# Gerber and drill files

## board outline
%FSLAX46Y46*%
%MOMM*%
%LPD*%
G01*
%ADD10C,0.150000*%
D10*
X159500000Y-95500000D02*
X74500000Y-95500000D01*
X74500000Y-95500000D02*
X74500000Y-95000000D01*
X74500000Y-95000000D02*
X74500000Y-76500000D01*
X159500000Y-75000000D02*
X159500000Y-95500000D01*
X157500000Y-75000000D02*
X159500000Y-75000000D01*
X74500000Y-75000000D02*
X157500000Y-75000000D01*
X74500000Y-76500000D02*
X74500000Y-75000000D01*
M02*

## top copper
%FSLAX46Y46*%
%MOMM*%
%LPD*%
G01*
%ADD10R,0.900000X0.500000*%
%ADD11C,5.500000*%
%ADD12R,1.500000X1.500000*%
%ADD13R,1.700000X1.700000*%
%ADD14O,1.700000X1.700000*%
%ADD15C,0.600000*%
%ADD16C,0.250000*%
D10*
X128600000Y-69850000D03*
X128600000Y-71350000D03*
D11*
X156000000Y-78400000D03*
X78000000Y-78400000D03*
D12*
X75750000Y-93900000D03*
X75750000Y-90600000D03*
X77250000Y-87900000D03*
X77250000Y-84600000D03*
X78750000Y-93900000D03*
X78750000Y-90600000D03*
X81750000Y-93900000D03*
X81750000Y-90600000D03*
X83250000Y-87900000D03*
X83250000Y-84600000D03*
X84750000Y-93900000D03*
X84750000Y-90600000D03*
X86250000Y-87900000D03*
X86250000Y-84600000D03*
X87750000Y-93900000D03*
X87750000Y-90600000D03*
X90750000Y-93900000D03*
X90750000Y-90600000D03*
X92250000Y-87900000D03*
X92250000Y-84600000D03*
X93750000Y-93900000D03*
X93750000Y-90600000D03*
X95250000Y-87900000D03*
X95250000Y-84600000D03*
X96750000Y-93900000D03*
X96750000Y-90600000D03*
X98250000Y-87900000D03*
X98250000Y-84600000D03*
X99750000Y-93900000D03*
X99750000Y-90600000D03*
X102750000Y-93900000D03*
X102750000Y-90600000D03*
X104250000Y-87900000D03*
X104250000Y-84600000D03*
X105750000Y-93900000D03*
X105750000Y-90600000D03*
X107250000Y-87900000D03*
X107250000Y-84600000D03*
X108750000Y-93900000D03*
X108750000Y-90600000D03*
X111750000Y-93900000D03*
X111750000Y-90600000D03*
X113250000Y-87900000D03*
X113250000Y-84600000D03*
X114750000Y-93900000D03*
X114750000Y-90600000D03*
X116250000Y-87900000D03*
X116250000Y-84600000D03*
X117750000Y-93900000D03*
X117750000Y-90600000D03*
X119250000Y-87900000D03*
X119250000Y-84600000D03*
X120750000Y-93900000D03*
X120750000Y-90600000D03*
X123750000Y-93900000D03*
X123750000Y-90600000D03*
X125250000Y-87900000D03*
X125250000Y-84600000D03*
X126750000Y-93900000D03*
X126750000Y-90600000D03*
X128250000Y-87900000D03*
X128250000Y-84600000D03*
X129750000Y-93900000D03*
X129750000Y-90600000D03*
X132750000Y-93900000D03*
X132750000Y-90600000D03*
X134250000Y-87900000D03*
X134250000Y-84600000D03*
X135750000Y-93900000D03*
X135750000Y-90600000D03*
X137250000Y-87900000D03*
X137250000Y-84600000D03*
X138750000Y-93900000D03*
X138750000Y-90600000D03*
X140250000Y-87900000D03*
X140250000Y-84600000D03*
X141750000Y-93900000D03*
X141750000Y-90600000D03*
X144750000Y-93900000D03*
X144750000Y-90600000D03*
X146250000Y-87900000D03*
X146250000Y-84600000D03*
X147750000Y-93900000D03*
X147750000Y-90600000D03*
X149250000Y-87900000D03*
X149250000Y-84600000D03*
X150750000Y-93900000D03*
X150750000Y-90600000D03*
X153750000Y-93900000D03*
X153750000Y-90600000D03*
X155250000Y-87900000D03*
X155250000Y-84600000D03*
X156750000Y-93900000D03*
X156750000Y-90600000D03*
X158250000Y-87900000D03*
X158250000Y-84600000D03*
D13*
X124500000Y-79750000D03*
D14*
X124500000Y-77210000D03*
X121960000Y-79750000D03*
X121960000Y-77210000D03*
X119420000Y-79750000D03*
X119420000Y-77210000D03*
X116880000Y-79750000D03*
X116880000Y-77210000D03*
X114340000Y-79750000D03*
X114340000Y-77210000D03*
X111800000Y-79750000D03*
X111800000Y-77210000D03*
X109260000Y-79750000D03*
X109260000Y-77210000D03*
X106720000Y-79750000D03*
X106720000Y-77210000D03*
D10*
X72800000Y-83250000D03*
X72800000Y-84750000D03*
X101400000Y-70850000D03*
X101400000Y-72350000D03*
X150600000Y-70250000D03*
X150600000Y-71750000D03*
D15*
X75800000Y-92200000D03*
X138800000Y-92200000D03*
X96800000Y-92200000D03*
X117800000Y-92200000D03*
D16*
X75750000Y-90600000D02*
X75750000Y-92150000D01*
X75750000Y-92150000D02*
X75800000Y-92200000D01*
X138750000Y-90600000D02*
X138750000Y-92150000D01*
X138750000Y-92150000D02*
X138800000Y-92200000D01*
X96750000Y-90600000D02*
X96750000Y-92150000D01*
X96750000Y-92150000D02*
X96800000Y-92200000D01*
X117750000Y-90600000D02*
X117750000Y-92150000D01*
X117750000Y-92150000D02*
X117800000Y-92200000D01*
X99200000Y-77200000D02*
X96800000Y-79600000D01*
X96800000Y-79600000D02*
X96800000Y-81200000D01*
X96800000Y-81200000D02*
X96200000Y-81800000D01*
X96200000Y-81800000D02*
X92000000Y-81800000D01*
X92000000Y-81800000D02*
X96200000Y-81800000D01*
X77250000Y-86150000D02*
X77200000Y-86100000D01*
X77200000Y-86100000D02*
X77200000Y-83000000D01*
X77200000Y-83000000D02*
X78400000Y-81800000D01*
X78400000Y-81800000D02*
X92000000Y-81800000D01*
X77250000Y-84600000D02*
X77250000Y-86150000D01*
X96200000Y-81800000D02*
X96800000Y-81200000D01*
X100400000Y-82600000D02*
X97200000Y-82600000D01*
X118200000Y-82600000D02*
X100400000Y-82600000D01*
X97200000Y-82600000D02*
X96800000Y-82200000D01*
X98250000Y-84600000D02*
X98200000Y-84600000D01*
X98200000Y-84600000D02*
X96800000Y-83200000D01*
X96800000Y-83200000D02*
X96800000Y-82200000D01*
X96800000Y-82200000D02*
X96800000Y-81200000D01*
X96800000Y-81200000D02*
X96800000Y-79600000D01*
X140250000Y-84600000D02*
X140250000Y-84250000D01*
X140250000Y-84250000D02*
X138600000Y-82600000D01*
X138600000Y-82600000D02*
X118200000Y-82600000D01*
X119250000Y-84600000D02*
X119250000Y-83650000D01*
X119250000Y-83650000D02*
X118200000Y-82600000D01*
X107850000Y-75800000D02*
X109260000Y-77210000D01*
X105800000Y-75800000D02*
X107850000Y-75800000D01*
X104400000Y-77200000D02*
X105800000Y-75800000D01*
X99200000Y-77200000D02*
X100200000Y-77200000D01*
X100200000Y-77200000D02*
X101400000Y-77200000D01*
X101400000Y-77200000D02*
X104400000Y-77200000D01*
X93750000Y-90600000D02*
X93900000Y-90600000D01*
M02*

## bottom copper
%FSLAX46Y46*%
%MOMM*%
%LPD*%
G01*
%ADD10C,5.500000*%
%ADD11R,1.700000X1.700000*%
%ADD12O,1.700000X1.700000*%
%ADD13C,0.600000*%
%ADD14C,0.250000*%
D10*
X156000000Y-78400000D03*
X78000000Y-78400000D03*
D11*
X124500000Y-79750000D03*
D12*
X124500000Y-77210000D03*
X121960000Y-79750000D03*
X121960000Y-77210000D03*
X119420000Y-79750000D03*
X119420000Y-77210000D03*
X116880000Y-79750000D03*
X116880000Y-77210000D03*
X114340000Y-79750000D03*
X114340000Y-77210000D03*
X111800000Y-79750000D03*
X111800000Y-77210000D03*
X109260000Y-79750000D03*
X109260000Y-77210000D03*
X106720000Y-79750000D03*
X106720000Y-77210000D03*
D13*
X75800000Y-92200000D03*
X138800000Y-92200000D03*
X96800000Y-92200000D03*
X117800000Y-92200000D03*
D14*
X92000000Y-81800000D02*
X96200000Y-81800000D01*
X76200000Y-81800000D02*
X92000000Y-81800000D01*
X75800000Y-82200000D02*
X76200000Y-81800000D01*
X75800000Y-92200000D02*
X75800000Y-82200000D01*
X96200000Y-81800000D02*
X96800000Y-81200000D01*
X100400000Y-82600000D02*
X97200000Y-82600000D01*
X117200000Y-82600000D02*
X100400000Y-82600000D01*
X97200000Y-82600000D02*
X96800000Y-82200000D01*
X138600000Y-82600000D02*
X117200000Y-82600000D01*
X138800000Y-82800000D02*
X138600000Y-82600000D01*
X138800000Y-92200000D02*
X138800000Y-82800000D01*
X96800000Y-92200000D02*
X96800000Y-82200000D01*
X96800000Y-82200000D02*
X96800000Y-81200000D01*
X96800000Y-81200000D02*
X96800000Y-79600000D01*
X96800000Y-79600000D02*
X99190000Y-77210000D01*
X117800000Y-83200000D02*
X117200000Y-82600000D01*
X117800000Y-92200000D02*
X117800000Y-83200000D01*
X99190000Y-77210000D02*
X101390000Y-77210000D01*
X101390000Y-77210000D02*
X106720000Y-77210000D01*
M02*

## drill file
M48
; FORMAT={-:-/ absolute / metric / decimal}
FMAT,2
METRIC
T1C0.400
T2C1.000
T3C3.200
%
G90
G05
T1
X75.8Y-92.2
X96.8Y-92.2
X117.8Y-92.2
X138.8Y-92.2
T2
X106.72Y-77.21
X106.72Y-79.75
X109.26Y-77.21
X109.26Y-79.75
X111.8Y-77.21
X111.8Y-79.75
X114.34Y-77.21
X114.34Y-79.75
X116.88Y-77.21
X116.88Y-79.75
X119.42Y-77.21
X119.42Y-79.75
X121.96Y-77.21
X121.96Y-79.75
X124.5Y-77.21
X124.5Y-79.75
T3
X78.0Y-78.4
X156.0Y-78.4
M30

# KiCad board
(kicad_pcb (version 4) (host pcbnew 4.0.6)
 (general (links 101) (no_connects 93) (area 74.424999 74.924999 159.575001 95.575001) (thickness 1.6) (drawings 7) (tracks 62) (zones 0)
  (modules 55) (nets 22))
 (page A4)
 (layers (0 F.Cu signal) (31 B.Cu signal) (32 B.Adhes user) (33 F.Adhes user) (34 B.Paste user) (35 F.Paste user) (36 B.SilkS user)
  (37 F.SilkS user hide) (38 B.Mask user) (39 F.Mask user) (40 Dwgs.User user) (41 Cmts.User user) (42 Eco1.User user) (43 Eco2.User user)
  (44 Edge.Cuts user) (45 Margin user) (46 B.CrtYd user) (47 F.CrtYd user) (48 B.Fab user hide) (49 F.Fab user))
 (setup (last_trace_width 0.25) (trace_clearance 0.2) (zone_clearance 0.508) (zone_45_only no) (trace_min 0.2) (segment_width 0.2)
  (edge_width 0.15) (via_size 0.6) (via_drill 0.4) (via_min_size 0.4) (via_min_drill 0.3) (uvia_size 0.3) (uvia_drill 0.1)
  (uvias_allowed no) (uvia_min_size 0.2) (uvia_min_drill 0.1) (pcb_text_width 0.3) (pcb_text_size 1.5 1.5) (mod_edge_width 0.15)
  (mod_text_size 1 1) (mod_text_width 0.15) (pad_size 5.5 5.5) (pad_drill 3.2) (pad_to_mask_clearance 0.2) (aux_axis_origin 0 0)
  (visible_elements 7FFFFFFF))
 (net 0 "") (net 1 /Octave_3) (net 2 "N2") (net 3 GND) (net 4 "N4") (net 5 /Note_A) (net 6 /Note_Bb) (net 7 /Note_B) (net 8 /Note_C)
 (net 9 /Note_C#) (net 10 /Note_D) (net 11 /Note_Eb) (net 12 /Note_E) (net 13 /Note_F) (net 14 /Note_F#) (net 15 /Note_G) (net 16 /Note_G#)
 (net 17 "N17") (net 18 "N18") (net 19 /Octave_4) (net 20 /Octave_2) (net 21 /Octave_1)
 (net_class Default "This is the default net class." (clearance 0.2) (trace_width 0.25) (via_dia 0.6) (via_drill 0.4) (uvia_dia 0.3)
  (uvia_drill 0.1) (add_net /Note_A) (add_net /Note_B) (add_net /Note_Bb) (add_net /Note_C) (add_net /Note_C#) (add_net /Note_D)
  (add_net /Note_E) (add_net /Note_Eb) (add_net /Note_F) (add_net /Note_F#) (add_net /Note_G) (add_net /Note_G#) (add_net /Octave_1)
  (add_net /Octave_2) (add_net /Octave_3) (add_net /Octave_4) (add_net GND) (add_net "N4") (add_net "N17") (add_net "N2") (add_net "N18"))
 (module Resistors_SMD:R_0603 (layer F.Cu) (at 128.6 70.6 270)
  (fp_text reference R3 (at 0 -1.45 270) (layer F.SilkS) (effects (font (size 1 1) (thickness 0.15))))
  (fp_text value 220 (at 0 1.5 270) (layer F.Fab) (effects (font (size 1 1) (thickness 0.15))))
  (pad 1 smd rect (at -0.75 0 270) (size 0.5 0.9) (layers F.Cu F.Paste F.Mask) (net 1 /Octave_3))
  (pad 2 smd rect (at 0.75 0 270) (size 0.5 0.9) (layers F.Cu F.Paste F.Mask) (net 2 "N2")))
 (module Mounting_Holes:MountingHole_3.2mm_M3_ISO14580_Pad (layer F.Cu) (at 156 78.4)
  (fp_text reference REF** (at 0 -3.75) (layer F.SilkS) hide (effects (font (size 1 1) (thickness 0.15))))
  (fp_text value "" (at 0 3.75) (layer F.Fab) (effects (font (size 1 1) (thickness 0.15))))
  (pad 1 thru_hole circle (at 0 0) (size 5.5 5.5) (drill 3.2) (layers *.Cu *.Mask) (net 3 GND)))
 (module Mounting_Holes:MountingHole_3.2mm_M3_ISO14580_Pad (layer F.Cu) (at 78 78.4)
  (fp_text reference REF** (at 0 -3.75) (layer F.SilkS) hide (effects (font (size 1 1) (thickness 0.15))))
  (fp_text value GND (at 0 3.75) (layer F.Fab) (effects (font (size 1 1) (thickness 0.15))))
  (pad 1 thru_hole circle (at 0 0) (size 5.5 5.5) (drill 3.2) (layers *.Cu *.Mask) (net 3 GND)))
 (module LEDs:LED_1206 (layer F.Cu) (at 75.75 92.25 270)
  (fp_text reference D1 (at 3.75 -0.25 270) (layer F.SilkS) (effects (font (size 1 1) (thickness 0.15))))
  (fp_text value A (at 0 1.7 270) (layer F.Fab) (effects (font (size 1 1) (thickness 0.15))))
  (pad 2 smd rect (at 1.65 0 90) (size 1.5 1.5) (layers F.Cu F.Paste F.Mask) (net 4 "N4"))
  (pad 1 smd rect (at -1.65 0 90) (size 1.5 1.5) (layers F.Cu F.Paste F.Mask) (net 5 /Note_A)))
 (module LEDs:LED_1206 (layer F.Cu) (at 77.25 86.25 270)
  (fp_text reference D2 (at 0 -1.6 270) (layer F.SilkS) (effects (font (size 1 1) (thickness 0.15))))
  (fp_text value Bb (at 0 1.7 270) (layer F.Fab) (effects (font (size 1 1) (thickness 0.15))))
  (pad 2 smd rect (at 1.65 0 90) (size 1.5 1.5) (layers F.Cu F.Paste F.Mask) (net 4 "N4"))
  (pad 1 smd rect (at -1.65 0 90) (size 1.5 1.5) (layers F.Cu F.Paste F.Mask) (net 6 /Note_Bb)))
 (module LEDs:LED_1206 (layer F.Cu) (at 78.75 92.25 270)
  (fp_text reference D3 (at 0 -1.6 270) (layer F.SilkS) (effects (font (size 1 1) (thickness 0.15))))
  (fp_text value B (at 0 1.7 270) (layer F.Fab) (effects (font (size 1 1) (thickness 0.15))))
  (pad 2 smd rect (at 1.65 0 90) (size 1.5 1.5) (layers F.Cu F.Paste F.Mask) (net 4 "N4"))
  (pad 1 smd rect (at -1.65 0 90) (size 1.5 1.5) (layers F.Cu F.Paste F.Mask) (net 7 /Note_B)))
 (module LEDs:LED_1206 (layer F.Cu) (at 81.75 92.25 270)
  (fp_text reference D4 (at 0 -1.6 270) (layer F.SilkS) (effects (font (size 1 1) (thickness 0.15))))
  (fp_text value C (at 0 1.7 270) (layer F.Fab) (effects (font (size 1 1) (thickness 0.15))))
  (pad 2 smd rect (at 1.65 0 90) (size 1.5 1.5) (layers F.Cu F.Paste F.Mask) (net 4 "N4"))
  (pad 1 smd rect (at -1.65 0 90) (size 1.5 1.5) (layers F.Cu F.Paste F.Mask) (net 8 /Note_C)))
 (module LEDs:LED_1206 (layer F.Cu) (at 83.25 86.25 270)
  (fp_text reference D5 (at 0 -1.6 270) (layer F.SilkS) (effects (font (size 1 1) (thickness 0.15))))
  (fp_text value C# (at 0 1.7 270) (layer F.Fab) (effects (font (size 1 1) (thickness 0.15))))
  (pad 2 smd rect (at 1.65 0 90) (size 1.5 1.5) (layers F.Cu F.Paste F.Mask) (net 4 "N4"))
  (pad 1 smd rect (at -1.65 0 90) (size 1.5 1.5) (layers F.Cu F.Paste F.Mask) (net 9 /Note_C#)))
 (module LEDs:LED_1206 (layer F.Cu) (at 84.75 92.25 270)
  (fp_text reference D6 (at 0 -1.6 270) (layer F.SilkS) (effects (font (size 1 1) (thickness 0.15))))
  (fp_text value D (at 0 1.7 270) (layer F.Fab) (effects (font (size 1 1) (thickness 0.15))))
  (pad 2 smd rect (at 1.65 0 90) (size 1.5 1.5) (layers F.Cu F.Paste F.Mask) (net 4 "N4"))
  (pad 1 smd rect (at -1.65 0 90) (size 1.5 1.5) (layers F.Cu F.Paste F.Mask) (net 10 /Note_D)))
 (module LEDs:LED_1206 (layer F.Cu) (at 86.25 86.25 270)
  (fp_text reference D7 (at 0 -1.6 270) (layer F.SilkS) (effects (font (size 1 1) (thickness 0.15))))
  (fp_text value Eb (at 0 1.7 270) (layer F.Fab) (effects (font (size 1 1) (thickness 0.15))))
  (pad 2 smd rect (at 1.65 0 90) (size 1.5 1.5) (layers F.Cu F.Paste F.Mask) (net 4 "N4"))
  (pad 1 smd rect (at -1.65 0 90) (size 1.5 1.5) (layers F.Cu F.Paste F.Mask) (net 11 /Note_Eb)))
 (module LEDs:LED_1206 (layer F.Cu) (at 87.75 92.25 270)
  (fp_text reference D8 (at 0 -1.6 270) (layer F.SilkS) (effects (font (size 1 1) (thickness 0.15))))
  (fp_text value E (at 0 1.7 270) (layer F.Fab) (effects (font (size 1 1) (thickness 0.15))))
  (pad 2 smd rect (at 1.65 0 90) (size 1.5 1.5) (layers F.Cu F.Paste F.Mask) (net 4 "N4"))
  (pad 1 smd rect (at -1.65 0 90) (size 1.5 1.5) (layers F.Cu F.Paste F.Mask) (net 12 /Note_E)))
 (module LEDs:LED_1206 (layer F.Cu) (at 90.75 92.25 270)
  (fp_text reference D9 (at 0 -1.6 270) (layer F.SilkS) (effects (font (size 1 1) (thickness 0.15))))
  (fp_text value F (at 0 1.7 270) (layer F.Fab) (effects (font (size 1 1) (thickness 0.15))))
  (pad 2 smd rect (at 1.65 0 90) (size 1.5 1.5) (layers F.Cu F.Paste F.Mask) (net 4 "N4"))
  (pad 1 smd rect (at -1.65 0 90) (size 1.5 1.5) (layers F.Cu F.Paste F.Mask) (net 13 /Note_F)))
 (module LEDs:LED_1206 (layer F.Cu) (at 92.25 86.25 270)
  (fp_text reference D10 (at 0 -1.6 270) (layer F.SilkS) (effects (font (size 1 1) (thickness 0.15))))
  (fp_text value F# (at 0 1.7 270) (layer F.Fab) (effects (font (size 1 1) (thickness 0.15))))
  (pad 2 smd rect (at 1.65 0 90) (size 1.5 1.5) (layers F.Cu F.Paste F.Mask) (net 4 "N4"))
  (pad 1 smd rect (at -1.65 0 90) (size 1.5 1.5) (layers F.Cu F.Paste F.Mask) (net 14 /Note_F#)))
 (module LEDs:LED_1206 (layer F.Cu) (at 93.75 92.25 270)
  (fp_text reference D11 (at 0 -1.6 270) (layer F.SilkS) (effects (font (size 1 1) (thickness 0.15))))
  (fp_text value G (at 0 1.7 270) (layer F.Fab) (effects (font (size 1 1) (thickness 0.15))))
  (pad 2 smd rect (at 1.65 0 90) (size 1.5 1.5) (layers F.Cu F.Paste F.Mask) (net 4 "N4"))
  (pad 1 smd rect (at -1.65 0 90) (size 1.5 1.5) (layers F.Cu F.Paste F.Mask) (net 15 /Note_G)))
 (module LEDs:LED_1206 (layer F.Cu) (at 95.25 86.25 270)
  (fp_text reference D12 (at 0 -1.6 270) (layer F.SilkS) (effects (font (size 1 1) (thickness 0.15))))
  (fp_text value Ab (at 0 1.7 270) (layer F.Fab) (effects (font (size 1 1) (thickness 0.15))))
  (pad 2 smd rect (at 1.65 0 90) (size 1.5 1.5) (layers F.Cu F.Paste F.Mask) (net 4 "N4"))
  (pad 1 smd rect (at -1.65 0 90) (size 1.5 1.5) (layers F.Cu F.Paste F.Mask) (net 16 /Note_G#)))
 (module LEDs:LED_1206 (layer F.Cu) (at 96.75 92.25 270)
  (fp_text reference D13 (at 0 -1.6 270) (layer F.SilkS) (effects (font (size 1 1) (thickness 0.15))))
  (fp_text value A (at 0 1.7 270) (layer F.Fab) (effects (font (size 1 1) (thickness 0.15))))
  (pad 2 smd rect (at 1.65 0 90) (size 1.5 1.5) (layers F.Cu F.Paste F.Mask) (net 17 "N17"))
  (pad 1 smd rect (at -1.65 0 90) (size 1.5 1.5) (layers F.Cu F.Paste F.Mask) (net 5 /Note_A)))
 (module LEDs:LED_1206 (layer F.Cu) (at 98.25 86.25 270)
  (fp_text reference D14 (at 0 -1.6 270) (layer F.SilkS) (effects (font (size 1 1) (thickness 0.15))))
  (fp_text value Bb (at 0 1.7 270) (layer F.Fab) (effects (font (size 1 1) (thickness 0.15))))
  (pad 2 smd rect (at 1.65 0 90) (size 1.5 1.5) (layers F.Cu F.Paste F.Mask) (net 17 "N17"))
  (pad 1 smd rect (at -1.65 0 90) (size 1.5 1.5) (layers F.Cu F.Paste F.Mask) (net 6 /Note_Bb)))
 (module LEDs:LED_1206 (layer F.Cu) (at 99.75 92.25 270)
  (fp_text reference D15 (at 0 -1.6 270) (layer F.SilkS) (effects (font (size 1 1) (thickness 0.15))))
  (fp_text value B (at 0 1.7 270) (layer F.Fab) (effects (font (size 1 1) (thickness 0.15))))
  (pad 2 smd rect (at 1.65 0 90) (size 1.5 1.5) (layers F.Cu F.Paste F.Mask) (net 17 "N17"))
  (pad 1 smd rect (at -1.65 0 90) (size 1.5 1.5) (layers F.Cu F.Paste F.Mask) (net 7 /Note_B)))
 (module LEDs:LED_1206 (layer F.Cu) (at 102.75 92.25 270)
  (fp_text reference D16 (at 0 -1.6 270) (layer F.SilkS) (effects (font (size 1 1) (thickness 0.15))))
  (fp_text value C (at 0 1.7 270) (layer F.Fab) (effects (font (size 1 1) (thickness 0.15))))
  (pad 2 smd rect (at 1.65 0 90) (size 1.5 1.5) (layers F.Cu F.Paste F.Mask) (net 17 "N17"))
  (pad 1 smd rect (at -1.65 0 90) (size 1.5 1.5) (layers F.Cu F.Paste F.Mask) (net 8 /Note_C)))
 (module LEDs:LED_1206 (layer F.Cu) (at 104.25 86.25 270)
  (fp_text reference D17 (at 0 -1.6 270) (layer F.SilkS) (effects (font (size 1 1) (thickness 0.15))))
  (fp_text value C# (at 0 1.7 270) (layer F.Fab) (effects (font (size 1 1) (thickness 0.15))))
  (pad 2 smd rect (at 1.65 0 90) (size 1.5 1.5) (layers F.Cu F.Paste F.Mask) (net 17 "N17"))
  (pad 1 smd rect (at -1.65 0 90) (size 1.5 1.5) (layers F.Cu F.Paste F.Mask) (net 9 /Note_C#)))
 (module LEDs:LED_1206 (layer F.Cu) (at 105.75 92.25 270)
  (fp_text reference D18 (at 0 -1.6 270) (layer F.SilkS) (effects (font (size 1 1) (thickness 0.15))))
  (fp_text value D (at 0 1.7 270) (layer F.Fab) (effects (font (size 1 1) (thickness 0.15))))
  (pad 2 smd rect (at 1.65 0 90) (size 1.5 1.5) (layers F.Cu F.Paste F.Mask) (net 17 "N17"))
  (pad 1 smd rect (at -1.65 0 90) (size 1.5 1.5) (layers F.Cu F.Paste F.Mask) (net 10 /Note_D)))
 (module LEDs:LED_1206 (layer F.Cu) (at 107.25 86.25 270)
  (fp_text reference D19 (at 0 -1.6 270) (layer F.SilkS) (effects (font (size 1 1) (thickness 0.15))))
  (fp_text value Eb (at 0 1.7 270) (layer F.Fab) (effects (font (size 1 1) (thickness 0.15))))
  (pad 2 smd rect (at 1.65 0 90) (size 1.5 1.5) (layers F.Cu F.Paste F.Mask) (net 17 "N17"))
  (pad 1 smd rect (at -1.65 0 90) (size 1.5 1.5) (layers F.Cu F.Paste F.Mask) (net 11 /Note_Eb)))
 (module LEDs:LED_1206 (layer F.Cu) (at 108.75 92.25 270)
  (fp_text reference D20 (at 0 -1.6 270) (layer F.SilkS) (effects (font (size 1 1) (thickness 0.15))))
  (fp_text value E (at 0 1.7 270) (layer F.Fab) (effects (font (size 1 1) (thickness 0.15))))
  (pad 2 smd rect (at 1.65 0 90) (size 1.5 1.5) (layers F.Cu F.Paste F.Mask) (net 17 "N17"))
  (pad 1 smd rect (at -1.65 0 90) (size 1.5 1.5) (layers F.Cu F.Paste F.Mask) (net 12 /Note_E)))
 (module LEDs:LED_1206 (layer F.Cu) (at 111.75 92.25 270)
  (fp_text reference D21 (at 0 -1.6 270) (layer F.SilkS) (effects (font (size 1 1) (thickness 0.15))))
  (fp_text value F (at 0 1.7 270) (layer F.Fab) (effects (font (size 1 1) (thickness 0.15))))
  (pad 2 smd rect (at 1.65 0 90) (size 1.5 1.5) (layers F.Cu F.Paste F.Mask) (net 17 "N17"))
  (pad 1 smd rect (at -1.65 0 90) (size 1.5 1.5) (layers F.Cu F.Paste F.Mask) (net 13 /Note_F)))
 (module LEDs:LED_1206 (layer F.Cu) (at 113.25 86.25 270)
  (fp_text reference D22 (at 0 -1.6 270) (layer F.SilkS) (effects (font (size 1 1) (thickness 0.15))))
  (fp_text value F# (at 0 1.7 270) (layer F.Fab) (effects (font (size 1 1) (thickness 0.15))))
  (pad 2 smd rect (at 1.65 0 90) (size 1.5 1.5) (layers F.Cu F.Paste F.Mask) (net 17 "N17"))
  (pad 1 smd rect (at -1.65 0 90) (size 1.5 1.5) (layers F.Cu F.Paste F.Mask) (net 14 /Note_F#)))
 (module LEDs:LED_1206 (layer F.Cu) (at 114.75 92.25 270)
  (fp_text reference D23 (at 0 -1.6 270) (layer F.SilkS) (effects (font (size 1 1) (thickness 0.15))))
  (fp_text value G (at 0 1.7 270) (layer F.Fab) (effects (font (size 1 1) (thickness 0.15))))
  (pad 2 smd rect (at 1.65 0 90) (size 1.5 1.5) (layers F.Cu F.Paste F.Mask) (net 17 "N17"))
  (pad 1 smd rect (at -1.65 0 90) (size 1.5 1.5) (layers F.Cu F.Paste F.Mask) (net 15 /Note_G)))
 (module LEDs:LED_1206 (layer F.Cu) (at 116.25 86.25 270)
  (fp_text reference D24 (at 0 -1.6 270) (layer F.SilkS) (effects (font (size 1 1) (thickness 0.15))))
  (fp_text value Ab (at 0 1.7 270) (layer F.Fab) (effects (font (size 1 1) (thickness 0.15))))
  (pad 2 smd rect (at 1.65 0 90) (size 1.5 1.5) (layers F.Cu F.Paste F.Mask) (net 17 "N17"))
  (pad 1 smd rect (at -1.65 0 90) (size 1.5 1.5) (layers F.Cu F.Paste F.Mask) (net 16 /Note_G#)))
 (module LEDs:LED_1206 (layer F.Cu) (at 117.75 92.25 270)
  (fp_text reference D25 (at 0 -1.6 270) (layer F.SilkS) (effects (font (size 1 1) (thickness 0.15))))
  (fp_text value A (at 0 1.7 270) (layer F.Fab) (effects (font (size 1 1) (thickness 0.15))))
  (pad 2 smd rect (at 1.65 0 90) (size 1.5 1.5) (layers F.Cu F.Paste F.Mask) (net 2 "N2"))
  (pad 1 smd rect (at -1.65 0 90) (size 1.5 1.5) (layers F.Cu F.Paste F.Mask) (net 5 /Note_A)))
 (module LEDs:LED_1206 (layer F.Cu) (at 119.25 86.25 270)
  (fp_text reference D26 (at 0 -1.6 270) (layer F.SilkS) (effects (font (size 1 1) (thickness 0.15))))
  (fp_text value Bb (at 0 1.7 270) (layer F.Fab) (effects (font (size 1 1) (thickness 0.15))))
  (pad 2 smd rect (at 1.65 0 90) (size 1.5 1.5) (layers F.Cu F.Paste F.Mask) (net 2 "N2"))
  (pad 1 smd rect (at -1.65 0 90) (size 1.5 1.5) (layers F.Cu F.Paste F.Mask) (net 6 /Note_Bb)))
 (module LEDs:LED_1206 (layer F.Cu) (at 120.75 92.25 270)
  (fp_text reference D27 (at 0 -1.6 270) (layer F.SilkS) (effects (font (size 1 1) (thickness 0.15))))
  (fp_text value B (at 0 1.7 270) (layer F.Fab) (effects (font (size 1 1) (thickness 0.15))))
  (pad 2 smd rect (at 1.65 0 90) (size 1.5 1.5) (layers F.Cu F.Paste F.Mask) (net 2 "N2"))
  (pad 1 smd rect (at -1.65 0 90) (size 1.5 1.5) (layers F.Cu F.Paste F.Mask) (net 7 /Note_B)))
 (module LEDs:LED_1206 (layer F.Cu) (at 123.75 92.25 270)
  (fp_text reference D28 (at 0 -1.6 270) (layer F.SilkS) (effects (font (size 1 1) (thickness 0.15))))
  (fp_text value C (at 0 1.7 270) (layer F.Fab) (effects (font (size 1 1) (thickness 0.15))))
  (pad 2 smd rect (at 1.65 0 90) (size 1.5 1.5) (layers F.Cu F.Paste F.Mask) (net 2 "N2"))
  (pad 1 smd rect (at -1.65 0 90) (size 1.5 1.5) (layers F.Cu F.Paste F.Mask) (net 8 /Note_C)))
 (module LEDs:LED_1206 (layer F.Cu) (at 125.25 86.25 270)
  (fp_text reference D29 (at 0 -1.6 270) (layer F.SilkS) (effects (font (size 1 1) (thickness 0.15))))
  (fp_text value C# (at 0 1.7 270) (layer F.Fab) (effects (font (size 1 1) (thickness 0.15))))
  (pad 2 smd rect (at 1.65 0 90) (size 1.5 1.5) (layers F.Cu F.Paste F.Mask) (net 2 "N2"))
  (pad 1 smd rect (at -1.65 0 90) (size 1.5 1.5) (layers F.Cu F.Paste F.Mask) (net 9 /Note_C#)))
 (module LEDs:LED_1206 (layer F.Cu) (at 126.75 92.25 270)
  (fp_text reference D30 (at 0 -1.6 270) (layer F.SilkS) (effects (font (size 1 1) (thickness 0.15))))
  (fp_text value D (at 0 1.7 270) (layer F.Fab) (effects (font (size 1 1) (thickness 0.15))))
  (pad 2 smd rect (at 1.65 0 90) (size 1.5 1.5) (layers F.Cu F.Paste F.Mask) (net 2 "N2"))
  (pad 1 smd rect (at -1.65 0 90) (size 1.5 1.5) (layers F.Cu F.Paste F.Mask) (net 10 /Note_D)))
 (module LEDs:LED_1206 (layer F.Cu) (at 128.25 86.25 270)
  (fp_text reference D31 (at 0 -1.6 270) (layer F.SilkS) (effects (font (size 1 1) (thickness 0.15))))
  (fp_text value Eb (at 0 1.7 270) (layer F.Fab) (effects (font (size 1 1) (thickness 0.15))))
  (pad 2 smd rect (at 1.65 0 90) (size 1.5 1.5) (layers F.Cu F.Paste F.Mask) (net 2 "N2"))
  (pad 1 smd rect (at -1.65 0 90) (size 1.5 1.5) (layers F.Cu F.Paste F.Mask) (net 11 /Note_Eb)))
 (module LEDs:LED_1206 (layer F.Cu) (at 129.75 92.25 270)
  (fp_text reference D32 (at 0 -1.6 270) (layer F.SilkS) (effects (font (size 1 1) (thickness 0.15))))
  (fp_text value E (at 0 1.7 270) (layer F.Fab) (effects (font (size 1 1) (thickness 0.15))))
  (pad 2 smd rect (at 1.65 0 90) (size 1.5 1.5) (layers F.Cu F.Paste F.Mask) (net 2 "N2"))
  (pad 1 smd rect (at -1.65 0 90) (size 1.5 1.5) (layers F.Cu F.Paste F.Mask) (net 12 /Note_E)))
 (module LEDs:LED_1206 (layer F.Cu) (at 132.75 92.25 270)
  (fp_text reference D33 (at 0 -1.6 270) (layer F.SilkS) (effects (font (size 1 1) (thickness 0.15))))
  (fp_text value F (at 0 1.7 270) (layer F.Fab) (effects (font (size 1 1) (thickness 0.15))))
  (pad 2 smd rect (at 1.65 0 90) (size 1.5 1.5) (layers F.Cu F.Paste F.Mask) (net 2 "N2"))
  (pad 1 smd rect (at -1.65 0 90) (size 1.5 1.5) (layers F.Cu F.Paste F.Mask) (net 13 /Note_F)))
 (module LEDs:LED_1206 (layer F.Cu) (at 134.25 86.25 270)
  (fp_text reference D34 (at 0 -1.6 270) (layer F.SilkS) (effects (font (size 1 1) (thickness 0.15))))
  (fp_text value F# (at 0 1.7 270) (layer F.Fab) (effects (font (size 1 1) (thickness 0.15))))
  (pad 2 smd rect (at 1.65 0 90) (size 1.5 1.5) (layers F.Cu F.Paste F.Mask) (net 2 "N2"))
  (pad 1 smd rect (at -1.65 0 90) (size 1.5 1.5) (layers F.Cu F.Paste F.Mask) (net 14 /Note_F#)))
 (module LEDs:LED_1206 (layer F.Cu) (at 135.75 92.25 270)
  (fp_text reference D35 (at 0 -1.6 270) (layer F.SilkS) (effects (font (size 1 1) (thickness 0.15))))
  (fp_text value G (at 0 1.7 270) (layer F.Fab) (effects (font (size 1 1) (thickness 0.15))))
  (pad 2 smd rect (at 1.65 0 90) (size 1.5 1.5) (layers F.Cu F.Paste F.Mask) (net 2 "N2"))
  (pad 1 smd rect (at -1.65 0 90) (size 1.5 1.5) (layers F.Cu F.Paste F.Mask) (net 15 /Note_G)))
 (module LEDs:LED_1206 (layer F.Cu) (at 137.25 86.25 270)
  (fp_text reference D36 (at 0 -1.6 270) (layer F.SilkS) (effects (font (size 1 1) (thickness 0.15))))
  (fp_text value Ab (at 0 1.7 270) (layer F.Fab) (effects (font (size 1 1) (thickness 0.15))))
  (pad 2 smd rect (at 1.65 0 90) (size 1.5 1.5) (layers F.Cu F.Paste F.Mask) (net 2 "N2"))
  (pad 1 smd rect (at -1.65 0 90) (size 1.5 1.5) (layers F.Cu F.Paste F.Mask) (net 16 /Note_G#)))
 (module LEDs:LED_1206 (layer F.Cu) (at 138.75 92.25 270)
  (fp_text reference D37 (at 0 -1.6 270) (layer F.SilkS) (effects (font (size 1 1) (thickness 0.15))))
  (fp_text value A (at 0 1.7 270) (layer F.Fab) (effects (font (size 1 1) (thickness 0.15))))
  (pad 2 smd rect (at 1.65 0 90) (size 1.5 1.5) (layers F.Cu F.Paste F.Mask) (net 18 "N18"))
  (pad 1 smd rect (at -1.65 0 90) (size 1.5 1.5) (layers F.Cu F.Paste F.Mask) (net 5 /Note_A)))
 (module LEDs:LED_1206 (layer F.Cu) (at 140.25 86.25 270)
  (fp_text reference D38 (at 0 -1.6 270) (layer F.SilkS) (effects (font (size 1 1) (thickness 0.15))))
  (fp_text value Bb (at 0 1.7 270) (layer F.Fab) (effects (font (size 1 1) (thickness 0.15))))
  (pad 2 smd rect (at 1.65 0 90) (size 1.5 1.5) (layers F.Cu F.Paste F.Mask) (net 18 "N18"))
  (pad 1 smd rect (at -1.65 0 90) (size 1.5 1.5) (layers F.Cu F.Paste F.Mask) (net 6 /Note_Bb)))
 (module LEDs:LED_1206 (layer F.Cu) (at 141.75 92.25 270)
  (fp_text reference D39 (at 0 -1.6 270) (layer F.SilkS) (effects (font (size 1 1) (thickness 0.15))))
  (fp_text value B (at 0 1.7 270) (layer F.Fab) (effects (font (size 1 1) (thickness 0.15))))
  (pad 2 smd rect (at 1.65 0 90) (size 1.5 1.5) (layers F.Cu F.Paste F.Mask) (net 18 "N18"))
  (pad 1 smd rect (at -1.65 0 90) (size 1.5 1.5) (layers F.Cu F.Paste F.Mask) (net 7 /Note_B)))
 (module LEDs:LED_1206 (layer F.Cu) (at 144.75 92.25 270)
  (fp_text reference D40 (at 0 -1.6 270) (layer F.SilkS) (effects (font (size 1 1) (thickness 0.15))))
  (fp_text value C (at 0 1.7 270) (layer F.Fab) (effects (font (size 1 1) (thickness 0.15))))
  (pad 2 smd rect (at 1.65 0 90) (size 1.5 1.5) (layers F.Cu F.Paste F.Mask) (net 18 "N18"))
  (pad 1 smd rect (at -1.65 0 90) (size 1.5 1.5) (layers F.Cu F.Paste F.Mask) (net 8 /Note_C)))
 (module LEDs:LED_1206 (layer F.Cu) (at 146.25 86.25 270)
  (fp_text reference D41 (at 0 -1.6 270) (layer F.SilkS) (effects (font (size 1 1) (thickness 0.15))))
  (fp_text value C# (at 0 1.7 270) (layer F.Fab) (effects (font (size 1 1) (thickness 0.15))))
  (pad 2 smd rect (at 1.65 0 90) (size 1.5 1.5) (layers F.Cu F.Paste F.Mask) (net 18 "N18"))
  (pad 1 smd rect (at -1.65 0 90) (size 1.5 1.5) (layers F.Cu F.Paste F.Mask) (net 9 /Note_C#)))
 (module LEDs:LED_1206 (layer F.Cu) (at 147.75 92.25 270)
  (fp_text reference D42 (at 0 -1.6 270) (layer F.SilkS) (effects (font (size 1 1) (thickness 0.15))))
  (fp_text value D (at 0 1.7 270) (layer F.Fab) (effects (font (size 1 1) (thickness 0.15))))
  (pad 2 smd rect (at 1.65 0 90) (size 1.5 1.5) (layers F.Cu F.Paste F.Mask) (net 18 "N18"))
  (pad 1 smd rect (at -1.65 0 90) (size 1.5 1.5) (layers F.Cu F.Paste F.Mask) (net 10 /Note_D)))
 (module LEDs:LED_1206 (layer F.Cu) (at 149.25 86.25 270)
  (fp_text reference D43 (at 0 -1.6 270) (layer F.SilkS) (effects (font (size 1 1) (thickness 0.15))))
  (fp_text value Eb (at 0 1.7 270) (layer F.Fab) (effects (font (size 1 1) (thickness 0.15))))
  (pad 2 smd rect (at 1.65 0 90) (size 1.5 1.5) (layers F.Cu F.Paste F.Mask) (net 18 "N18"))
  (pad 1 smd rect (at -1.65 0 90) (size 1.5 1.5) (layers F.Cu F.Paste F.Mask) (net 11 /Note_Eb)))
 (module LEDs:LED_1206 (layer F.Cu) (at 150.75 92.25 270)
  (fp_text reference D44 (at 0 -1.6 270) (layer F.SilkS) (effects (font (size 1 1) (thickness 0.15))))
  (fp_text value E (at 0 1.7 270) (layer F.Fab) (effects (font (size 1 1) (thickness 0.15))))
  (pad 2 smd rect (at 1.65 0 90) (size 1.5 1.5) (layers F.Cu F.Paste F.Mask) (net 18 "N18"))
  (pad 1 smd rect (at -1.65 0 90) (size 1.5 1.5) (layers F.Cu F.Paste F.Mask) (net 12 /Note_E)))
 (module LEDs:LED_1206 (layer F.Cu) (at 153.75 92.25 270)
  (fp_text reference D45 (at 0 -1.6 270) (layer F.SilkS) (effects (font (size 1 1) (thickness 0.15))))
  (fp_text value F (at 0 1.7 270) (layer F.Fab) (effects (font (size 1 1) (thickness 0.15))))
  (pad 2 smd rect (at 1.65 0 90) (size 1.5 1.5) (layers F.Cu F.Paste F.Mask) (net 18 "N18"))
  (pad 1 smd rect (at -1.65 0 90) (size 1.5 1.5) (layers F.Cu F.Paste F.Mask) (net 13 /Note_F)))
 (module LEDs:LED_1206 (layer F.Cu) (at 155.25 86.25 270)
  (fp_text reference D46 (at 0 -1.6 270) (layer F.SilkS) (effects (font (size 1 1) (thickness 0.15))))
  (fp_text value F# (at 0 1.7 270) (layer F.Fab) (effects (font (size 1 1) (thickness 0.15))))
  (pad 2 smd rect (at 1.65 0 90) (size 1.5 1.5) (layers F.Cu F.Paste F.Mask) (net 18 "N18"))
  (pad 1 smd rect (at -1.65 0 90) (size 1.5 1.5) (layers F.Cu F.Paste F.Mask) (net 14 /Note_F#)))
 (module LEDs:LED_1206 (layer F.Cu) (at 156.75 92.25 270)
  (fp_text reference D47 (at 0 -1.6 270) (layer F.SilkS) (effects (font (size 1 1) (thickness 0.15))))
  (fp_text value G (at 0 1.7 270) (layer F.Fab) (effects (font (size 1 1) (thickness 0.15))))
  (pad 2 smd rect (at 1.65 0 90) (size 1.5 1.5) (layers F.Cu F.Paste F.Mask) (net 18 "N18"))
  (pad 1 smd rect (at -1.65 0 90) (size 1.5 1.5) (layers F.Cu F.Paste F.Mask) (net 15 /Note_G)))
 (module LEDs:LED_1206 (layer F.Cu) (at 158.25 86.25 270)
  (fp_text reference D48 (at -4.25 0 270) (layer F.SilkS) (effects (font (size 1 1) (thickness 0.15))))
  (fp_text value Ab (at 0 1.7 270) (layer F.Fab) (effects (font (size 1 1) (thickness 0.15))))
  (pad 2 smd rect (at 1.65 0 90) (size 1.5 1.5) (layers F.Cu F.Paste F.Mask) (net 18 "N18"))
  (pad 1 smd rect (at -1.65 0 90) (size 1.5 1.5) (layers F.Cu F.Paste F.Mask) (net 16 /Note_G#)))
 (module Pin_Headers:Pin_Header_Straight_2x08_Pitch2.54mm (layer B.Cu) (at 124.5 79.75 90)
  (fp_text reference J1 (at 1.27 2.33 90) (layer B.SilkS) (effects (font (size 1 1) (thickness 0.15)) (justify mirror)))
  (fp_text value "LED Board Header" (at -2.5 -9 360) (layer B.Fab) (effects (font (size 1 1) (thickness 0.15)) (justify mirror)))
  (pad 1 thru_hole rect (at 0 0 90) (size 1.7 1.7) (drill 1) (layers *.Cu *.Mask) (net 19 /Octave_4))
  (pad 2 thru_hole oval (at 2.54 0 90) (size 1.7 1.7) (drill 1) (layers *.Cu *.Mask) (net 12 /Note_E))
  (pad 3 thru_hole oval (at 0 -2.54 90) (size 1.7 1.7) (drill 1) (layers *.Cu *.Mask) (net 1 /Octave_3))
  (pad 4 thru_hole oval (at 2.54 -2.54 90) (size 1.7 1.7) (drill 1) (layers *.Cu *.Mask) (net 11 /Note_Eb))
  (pad 5 thru_hole oval (at 0 -5.08 90) (size 1.7 1.7) (drill 1) (layers *.Cu *.Mask) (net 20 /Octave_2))
  (pad 6 thru_hole oval (at 2.54 -5.08 90) (size 1.7 1.7) (drill 1) (layers *.Cu *.Mask) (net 10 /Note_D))
  (pad 7 thru_hole oval (at 0 -7.62 90) (size 1.7 1.7) (drill 1) (layers *.Cu *.Mask) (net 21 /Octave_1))
  (pad 8 thru_hole oval (at 2.54 -7.62 90) (size 1.7 1.7) (drill 1) (layers *.Cu *.Mask) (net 9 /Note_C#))
  (pad 9 thru_hole oval (at 0 -10.16 90) (size 1.7 1.7) (drill 1) (layers *.Cu *.Mask) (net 16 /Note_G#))
  (pad 10 thru_hole oval (at 2.54 -10.16 90) (size 1.7 1.7) (drill 1) (layers *.Cu *.Mask) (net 8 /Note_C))
  (pad 11 thru_hole oval (at 0 -12.7 90) (size 1.7 1.7) (drill 1) (layers *.Cu *.Mask) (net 15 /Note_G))
  (pad 12 thru_hole oval (at 2.54 -12.7 90) (size 1.7 1.7) (drill 1) (layers *.Cu *.Mask) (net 7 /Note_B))
  (pad 13 thru_hole oval (at 0 -15.24 90) (size 1.7 1.7) (drill 1) (layers *.Cu *.Mask) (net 14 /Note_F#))
  (pad 14 thru_hole oval (at 2.54 -15.24 90) (size 1.7 1.7) (drill 1) (layers *.Cu *.Mask) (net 6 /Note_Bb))
  (pad 15 thru_hole oval (at 0 -17.78 90) (size 1.7 1.7) (drill 1) (layers *.Cu *.Mask) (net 13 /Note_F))
  (pad 16 thru_hole oval (at 2.54 -17.78 90) (size 1.7 1.7) (drill 1) (layers *.Cu *.Mask) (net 5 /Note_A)))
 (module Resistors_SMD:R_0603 (layer F.Cu) (at 72.8 84 270)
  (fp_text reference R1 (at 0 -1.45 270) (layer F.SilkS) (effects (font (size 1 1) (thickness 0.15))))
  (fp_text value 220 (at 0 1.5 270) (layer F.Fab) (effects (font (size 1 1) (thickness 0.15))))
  (pad 1 smd rect (at -0.75 0 270) (size 0.5 0.9) (layers F.Cu F.Paste F.Mask) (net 21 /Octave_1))
  (pad 2 smd rect (at 0.75 0 270) (size 0.5 0.9) (layers F.Cu F.Paste F.Mask) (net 4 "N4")))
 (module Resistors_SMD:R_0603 (layer F.Cu) (at 101.4 71.6 270)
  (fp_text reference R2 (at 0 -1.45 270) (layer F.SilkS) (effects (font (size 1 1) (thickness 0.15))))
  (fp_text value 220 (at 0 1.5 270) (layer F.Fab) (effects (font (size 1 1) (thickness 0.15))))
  (pad 1 smd rect (at -0.75 0 270) (size 0.5 0.9) (layers F.Cu F.Paste F.Mask) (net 20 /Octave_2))
  (pad 2 smd rect (at 0.75 0 270) (size 0.5 0.9) (layers F.Cu F.Paste F.Mask) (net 17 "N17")))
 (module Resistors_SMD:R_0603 (layer F.Cu) (at 150.6 71 270)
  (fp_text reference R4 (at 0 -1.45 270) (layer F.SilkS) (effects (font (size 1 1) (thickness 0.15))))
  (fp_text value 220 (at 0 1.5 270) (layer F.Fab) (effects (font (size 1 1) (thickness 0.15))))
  (pad 1 smd rect (at -0.75 0 270) (size 0.5 0.9) (layers F.Cu F.Paste F.Mask) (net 19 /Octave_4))
  (pad 2 smd rect (at 0.75 0 270) (size 0.5 0.9) (layers F.Cu F.Paste F.Mask) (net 18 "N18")))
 (gr_line (start 159.5 95.5) (end 74.5 95.5) (angle 90) (layer Edge.Cuts) (width 0.15))
 (gr_line (start 74.5 95.5) (end 74.5 95) (angle 90) (layer Edge.Cuts) (width 0.15))
 (gr_line (start 74.5 95) (end 74.5 76.5) (angle 90) (layer Edge.Cuts) (width 0.15))
 (gr_line (start 159.5 75) (end 159.5 95.5) (angle 90) (layer Edge.Cuts) (width 0.15))
 (gr_line (start 157.5 75) (end 159.5 75) (angle 90) (layer Edge.Cuts) (width 0.15))
 (gr_line (start 74.5 75) (end 157.5 75) (angle 90) (layer Edge.Cuts) (width 0.15))
 (gr_line (start 74.5 76.5) (end 74.5 75) (angle 90) (layer Edge.Cuts) (width 0.15))
 (segment (start 92 81.8) (end 96.2 81.8) (width 0.25) (layer B.Cu) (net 5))
 (segment (start 75.75 90.6) (end 75.75 92.15) (width 0.25) (layer F.Cu) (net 5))
 (segment (start 76.2 81.8) (end 92 81.8) (width 0.25) (layer B.Cu) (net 5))
 (segment (start 75.8 82.2) (end 76.2 81.8) (width 0.25) (layer B.Cu) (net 5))
 (segment (start 75.8 92.2) (end 75.8 82.2) (width 0.25) (layer B.Cu) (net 5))
 (via (at 75.8 92.2) (size 0.6) (drill 0.4) (layers F.Cu B.Cu) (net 5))
 (segment (start 75.75 92.15) (end 75.8 92.2) (width 0.25) (layer F.Cu) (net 5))
 (segment (start 96.2 81.8) (end 96.8 81.2) (width 0.25) (layer B.Cu) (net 5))
 (segment (start 100.4 82.6) (end 97.2 82.6) (width 0.25) (layer B.Cu) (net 5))
 (segment (start 117.2 82.6) (end 100.4 82.6) (width 0.25) (layer B.Cu) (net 5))
 (segment (start 97.2 82.6) (end 96.8 82.2) (width 0.25) (layer B.Cu) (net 5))
 (segment (start 138.75 90.6) (end 138.75 92.15) (width 0.25) (layer F.Cu) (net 5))
 (segment (start 138.6 82.6) (end 117.2 82.6) (width 0.25) (layer B.Cu) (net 5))
 (segment (start 138.8 82.8) (end 138.6 82.6) (width 0.25) (layer B.Cu) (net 5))
 (segment (start 138.8 92.2) (end 138.8 82.8) (width 0.25) (layer B.Cu) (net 5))
 (via (at 138.8 92.2) (size 0.6) (drill 0.4) (layers F.Cu B.Cu) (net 5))
 (segment (start 138.75 92.15) (end 138.8 92.2) (width 0.25) (layer F.Cu) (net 5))
 (segment (start 96.8 92.2) (end 96.8 82.2) (width 0.25) (layer B.Cu) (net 5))
 (segment (start 96.75 90.6) (end 96.75 92.15) (width 0.25) (layer F.Cu) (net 5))
 (via (at 96.8 92.2) (size 0.6) (drill 0.4) (layers F.Cu B.Cu) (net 5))
 (segment (start 96.75 92.15) (end 96.8 92.2) (width 0.25) (layer F.Cu) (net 5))
 (segment (start 96.8 82.2) (end 96.8 81.2) (width 0.25) (layer B.Cu) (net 5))
 (segment (start 96.8 81.2) (end 96.8 79.6) (width 0.25) (layer B.Cu) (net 5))
 (segment (start 96.8 79.6) (end 99.19 77.21) (width 0.25) (layer B.Cu) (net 5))
 (segment (start 117.75 90.6) (end 117.75 92.15) (width 0.25) (layer F.Cu) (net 5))
 (segment (start 117.8 83.2) (end 117.2 82.6) (width 0.25) (layer B.Cu) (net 5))
 (segment (start 117.8 92.2) (end 117.8 83.2) (width 0.25) (layer B.Cu) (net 5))
 (via (at 117.8 92.2) (size 0.6) (drill 0.4) (layers F.Cu B.Cu) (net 5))
 (segment (start 117.75 92.15) (end 117.8 92.2) (width 0.25) (layer F.Cu) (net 5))
 (segment (start 99.19 77.21) (end 101.39 77.21) (width 0.25) (layer B.Cu) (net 5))
 (segment (start 101.39 77.21) (end 106.72 77.21) (width 0.25) (layer B.Cu) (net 5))
 (segment (start 99.2 77.2) (end 96.8 79.6) (width 0.25) (layer F.Cu) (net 6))
 (segment (start 96.8 79.6) (end 96.8 81.2) (width 0.25) (layer F.Cu) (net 6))
 (segment (start 96.8 81.2) (end 96.2 81.8) (width 0.25) (layer F.Cu) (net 6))
 (segment (start 96.2 81.8) (end 92 81.8) (width 0.25) (layer F.Cu) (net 6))
 (segment (start 92 81.8) (end 96.2 81.8) (width 0.25) (layer F.Cu) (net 6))
 (segment (start 77.25 86.15) (end 77.2 86.1) (width 0.25) (layer F.Cu) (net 6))
 (segment (start 77.2 86.1) (end 77.2 83) (width 0.25) (layer F.Cu) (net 6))
 (segment (start 77.2 83) (end 78.4 81.8) (width 0.25) (layer F.Cu) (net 6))
 (segment (start 78.4 81.8) (end 92 81.8) (width 0.25) (layer F.Cu) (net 6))
 (segment (start 77.25 84.6) (end 77.25 86.15) (width 0.25) (layer F.Cu) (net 6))
 (segment (start 96.2 81.8) (end 96.8 81.2) (width 0.25) (layer F.Cu) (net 6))
 (segment (start 100.4 82.6) (end 97.2 82.6) (width 0.25) (layer F.Cu) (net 6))
 (segment (start 118.2 82.6) (end 100.4 82.6) (width 0.25) (layer F.Cu) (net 6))
 (segment (start 97.2 82.6) (end 96.8 82.2) (width 0.25) (layer F.Cu) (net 6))
 (segment (start 98.25 84.6) (end 98.2 84.6) (width 0.25) (layer F.Cu) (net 6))
 (segment (start 98.2 84.6) (end 96.8 83.2) (width 0.25) (layer F.Cu) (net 6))
 (segment (start 96.8 83.2) (end 96.8 82.2) (width 0.25) (layer F.Cu) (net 6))
 (segment (start 96.8 82.2) (end 96.8 81.2) (width 0.25) (layer F.Cu) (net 6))
 (segment (start 96.8 81.2) (end 96.8 79.6) (width 0.25) (layer F.Cu) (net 6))
 (segment (start 140.25 84.6) (end 140.25 84.25) (width 0.25) (layer F.Cu) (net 6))
 (segment (start 140.25 84.25) (end 138.6 82.6) (width 0.25) (layer F.Cu) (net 6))
 (segment (start 138.6 82.6) (end 118.2 82.6) (width 0.25) (layer F.Cu) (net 6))
 (segment (start 119.25 84.6) (end 119.25 83.65) (width 0.25) (layer F.Cu) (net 6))
 (segment (start 119.25 83.65) (end 118.2 82.6) (width 0.25) (layer F.Cu) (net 6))
 (segment (start 107.85 75.8) (end 109.26 77.21) (width 0.25) (layer F.Cu) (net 6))
 (segment (start 105.8 75.8) (end 107.85 75.8) (width 0.25) (layer F.Cu) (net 6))
 (segment (start 104.4 77.2) (end 105.8 75.8) (width 0.25) (layer F.Cu) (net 6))
 (segment (start 99.2 77.2) (end 100.2 77.2) (width 0.25) (layer F.Cu) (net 6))
 (segment (start 100.2 77.2) (end 101.4 77.2) (width 0.25) (layer F.Cu) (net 6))
 (segment (start 101.4 77.2) (end 104.4 77.2) (width 0.25) (layer F.Cu) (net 6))
 (segment (start 93.75 90.6) (end 93.9 90.6) (width 0.25) (layer F.Cu) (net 15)))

